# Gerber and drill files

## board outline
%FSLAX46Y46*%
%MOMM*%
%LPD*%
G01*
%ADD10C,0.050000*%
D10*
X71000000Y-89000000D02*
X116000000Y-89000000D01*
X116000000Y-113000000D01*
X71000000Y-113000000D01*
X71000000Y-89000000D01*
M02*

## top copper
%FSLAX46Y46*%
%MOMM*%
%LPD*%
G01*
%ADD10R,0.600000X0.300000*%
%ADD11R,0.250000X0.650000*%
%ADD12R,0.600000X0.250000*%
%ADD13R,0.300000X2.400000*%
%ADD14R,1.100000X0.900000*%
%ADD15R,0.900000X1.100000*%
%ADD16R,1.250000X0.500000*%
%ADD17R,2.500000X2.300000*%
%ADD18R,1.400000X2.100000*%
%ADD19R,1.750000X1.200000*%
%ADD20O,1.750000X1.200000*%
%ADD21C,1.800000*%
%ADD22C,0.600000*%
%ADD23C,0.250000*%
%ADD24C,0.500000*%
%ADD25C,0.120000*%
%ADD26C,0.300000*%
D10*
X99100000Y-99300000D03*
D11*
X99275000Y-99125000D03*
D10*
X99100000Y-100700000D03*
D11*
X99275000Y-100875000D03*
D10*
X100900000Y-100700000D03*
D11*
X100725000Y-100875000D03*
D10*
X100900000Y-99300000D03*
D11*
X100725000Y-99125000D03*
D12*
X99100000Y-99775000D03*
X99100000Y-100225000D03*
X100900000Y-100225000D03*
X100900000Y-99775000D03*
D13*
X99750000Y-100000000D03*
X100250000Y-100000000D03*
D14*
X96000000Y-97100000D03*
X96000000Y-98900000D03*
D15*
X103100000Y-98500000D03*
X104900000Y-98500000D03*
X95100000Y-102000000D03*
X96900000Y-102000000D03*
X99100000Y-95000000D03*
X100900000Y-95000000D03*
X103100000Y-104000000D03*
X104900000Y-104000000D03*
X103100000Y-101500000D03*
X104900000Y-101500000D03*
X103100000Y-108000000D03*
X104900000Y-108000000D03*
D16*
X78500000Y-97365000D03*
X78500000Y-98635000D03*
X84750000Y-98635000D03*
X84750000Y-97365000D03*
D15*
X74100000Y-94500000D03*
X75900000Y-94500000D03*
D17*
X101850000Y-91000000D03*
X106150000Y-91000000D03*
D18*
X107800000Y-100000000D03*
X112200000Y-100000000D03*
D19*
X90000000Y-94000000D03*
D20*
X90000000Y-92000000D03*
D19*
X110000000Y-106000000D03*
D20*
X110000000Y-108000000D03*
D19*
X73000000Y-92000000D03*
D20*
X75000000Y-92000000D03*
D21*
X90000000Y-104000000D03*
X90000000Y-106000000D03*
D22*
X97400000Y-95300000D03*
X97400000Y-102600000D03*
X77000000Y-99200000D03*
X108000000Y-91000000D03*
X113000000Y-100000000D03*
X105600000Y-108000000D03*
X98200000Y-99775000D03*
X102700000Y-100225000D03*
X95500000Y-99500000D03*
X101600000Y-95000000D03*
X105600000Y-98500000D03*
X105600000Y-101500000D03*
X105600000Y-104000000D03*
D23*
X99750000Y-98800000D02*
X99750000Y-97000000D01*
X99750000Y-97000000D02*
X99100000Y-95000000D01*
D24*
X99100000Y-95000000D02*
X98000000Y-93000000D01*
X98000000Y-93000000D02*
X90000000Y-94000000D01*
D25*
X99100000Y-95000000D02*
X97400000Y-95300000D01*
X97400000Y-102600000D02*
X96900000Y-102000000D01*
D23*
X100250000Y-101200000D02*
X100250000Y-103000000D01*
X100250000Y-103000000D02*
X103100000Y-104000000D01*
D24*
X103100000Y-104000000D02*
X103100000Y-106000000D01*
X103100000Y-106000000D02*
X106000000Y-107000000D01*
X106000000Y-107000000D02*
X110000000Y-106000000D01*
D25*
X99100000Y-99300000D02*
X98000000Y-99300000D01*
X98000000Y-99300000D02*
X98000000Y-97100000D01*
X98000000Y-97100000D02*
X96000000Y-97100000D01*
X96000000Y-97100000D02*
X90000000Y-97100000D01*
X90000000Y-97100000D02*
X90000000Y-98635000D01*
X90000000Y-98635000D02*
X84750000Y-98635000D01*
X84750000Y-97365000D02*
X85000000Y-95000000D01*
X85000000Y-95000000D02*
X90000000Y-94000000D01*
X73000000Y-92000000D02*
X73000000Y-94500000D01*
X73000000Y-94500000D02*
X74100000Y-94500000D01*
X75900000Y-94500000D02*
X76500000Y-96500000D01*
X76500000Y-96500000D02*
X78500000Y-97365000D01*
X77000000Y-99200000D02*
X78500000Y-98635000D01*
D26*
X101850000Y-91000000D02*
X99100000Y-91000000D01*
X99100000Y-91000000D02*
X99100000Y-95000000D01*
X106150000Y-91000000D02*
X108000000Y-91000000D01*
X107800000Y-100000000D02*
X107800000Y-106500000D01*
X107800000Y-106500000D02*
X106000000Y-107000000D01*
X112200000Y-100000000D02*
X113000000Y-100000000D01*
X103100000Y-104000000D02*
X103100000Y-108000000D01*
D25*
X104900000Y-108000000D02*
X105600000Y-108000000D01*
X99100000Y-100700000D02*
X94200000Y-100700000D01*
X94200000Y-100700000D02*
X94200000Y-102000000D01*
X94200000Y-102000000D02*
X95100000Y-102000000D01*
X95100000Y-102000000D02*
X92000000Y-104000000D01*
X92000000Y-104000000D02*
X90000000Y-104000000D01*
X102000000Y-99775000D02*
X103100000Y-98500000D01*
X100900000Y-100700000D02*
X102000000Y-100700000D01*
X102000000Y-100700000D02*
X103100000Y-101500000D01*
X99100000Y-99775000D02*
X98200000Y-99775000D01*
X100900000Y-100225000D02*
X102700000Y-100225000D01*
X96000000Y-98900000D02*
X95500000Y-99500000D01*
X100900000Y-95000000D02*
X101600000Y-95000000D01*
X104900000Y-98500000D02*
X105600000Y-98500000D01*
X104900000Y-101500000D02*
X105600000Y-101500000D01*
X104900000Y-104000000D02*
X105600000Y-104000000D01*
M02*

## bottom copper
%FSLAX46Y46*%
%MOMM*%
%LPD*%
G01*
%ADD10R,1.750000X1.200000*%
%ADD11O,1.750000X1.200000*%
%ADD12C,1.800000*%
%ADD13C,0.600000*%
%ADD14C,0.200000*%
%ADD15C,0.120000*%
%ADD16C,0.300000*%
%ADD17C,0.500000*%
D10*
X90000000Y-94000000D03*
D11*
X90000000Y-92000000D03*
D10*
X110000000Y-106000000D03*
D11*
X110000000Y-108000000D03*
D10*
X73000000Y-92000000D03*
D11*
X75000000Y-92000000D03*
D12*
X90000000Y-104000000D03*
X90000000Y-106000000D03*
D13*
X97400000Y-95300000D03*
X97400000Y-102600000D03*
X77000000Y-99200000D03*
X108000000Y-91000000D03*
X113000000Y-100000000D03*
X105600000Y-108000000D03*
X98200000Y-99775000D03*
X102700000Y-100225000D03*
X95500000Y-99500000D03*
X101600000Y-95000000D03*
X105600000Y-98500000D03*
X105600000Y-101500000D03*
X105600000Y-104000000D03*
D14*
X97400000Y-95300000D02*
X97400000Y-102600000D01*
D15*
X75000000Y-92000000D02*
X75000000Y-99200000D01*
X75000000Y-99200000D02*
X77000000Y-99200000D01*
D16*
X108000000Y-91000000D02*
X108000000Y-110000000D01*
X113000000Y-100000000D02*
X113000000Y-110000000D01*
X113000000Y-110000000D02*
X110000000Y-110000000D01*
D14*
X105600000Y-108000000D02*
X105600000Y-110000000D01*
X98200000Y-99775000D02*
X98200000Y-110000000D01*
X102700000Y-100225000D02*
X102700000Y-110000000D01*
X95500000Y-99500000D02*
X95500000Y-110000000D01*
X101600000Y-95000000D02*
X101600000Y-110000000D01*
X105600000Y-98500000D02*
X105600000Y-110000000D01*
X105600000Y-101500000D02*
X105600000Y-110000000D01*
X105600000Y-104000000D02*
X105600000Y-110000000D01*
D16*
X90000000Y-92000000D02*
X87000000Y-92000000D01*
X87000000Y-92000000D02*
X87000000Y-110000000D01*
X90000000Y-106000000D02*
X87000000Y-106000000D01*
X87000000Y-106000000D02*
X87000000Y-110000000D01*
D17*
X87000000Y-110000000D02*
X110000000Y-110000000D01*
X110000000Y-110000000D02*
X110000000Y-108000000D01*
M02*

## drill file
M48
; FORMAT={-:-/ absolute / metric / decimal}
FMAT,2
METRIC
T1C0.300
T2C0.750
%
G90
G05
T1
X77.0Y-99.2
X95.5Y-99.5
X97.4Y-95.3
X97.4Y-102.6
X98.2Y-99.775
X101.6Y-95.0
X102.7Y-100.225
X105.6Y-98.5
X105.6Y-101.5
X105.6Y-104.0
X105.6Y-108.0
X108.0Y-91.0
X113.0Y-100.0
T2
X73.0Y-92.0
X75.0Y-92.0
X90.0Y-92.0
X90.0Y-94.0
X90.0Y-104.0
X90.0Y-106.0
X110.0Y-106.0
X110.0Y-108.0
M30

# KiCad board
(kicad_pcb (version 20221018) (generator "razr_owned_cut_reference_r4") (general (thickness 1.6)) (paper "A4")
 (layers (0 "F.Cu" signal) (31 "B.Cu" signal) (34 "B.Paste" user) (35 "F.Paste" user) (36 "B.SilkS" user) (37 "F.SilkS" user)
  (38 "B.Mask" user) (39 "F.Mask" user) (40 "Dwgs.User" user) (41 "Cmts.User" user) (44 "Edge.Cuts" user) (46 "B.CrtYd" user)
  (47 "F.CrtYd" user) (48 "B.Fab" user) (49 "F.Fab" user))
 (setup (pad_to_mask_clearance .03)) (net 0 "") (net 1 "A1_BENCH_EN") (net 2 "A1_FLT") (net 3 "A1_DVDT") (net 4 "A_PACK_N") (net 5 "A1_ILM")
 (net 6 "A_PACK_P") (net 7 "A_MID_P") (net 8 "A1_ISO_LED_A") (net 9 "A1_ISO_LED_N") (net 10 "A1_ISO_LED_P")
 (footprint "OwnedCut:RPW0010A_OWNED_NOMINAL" (layer "F.Cu") (at 100 100)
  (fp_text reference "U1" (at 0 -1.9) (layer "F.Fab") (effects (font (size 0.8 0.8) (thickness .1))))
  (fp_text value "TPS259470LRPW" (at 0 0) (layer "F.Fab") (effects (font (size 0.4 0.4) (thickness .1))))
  (pad "1" smd rect (at -0.9 -0.7) (size 0.6 0.3) (layers "F.Cu" "F.Paste" "F.Mask") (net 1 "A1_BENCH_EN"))
  (pad "1" smd rect (at -0.725 -0.875) (size 0.25 0.65) (layers "F.Cu" "F.Paste" "F.Mask") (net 1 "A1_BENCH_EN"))
  (pad "4" smd rect (at -0.9 0.7) (size 0.6 0.3) (layers "F.Cu" "F.Paste" "F.Mask") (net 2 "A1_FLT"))
  (pad "4" smd rect (at -0.725 0.875) (size 0.25 0.65) (layers "F.Cu" "F.Paste" "F.Mask") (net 2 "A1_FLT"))
  (pad "7" smd rect (at 0.9 0.7) (size 0.6 0.3) (layers "F.Cu" "F.Paste" "F.Mask") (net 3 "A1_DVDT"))
  (pad "7" smd rect (at 0.725 0.875) (size 0.25 0.65) (layers "F.Cu" "F.Paste" "F.Mask") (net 3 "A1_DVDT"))
  (pad "10" smd rect (at 0.9 -0.7) (size 0.6 0.3) (layers "F.Cu" "F.Paste" "F.Mask"))
  (pad "10" smd rect (at 0.725 -0.875) (size 0.25 0.65) (layers "F.Cu" "F.Paste" "F.Mask"))
  (pad "2" smd rect (at -0.9 -0.225) (size 0.6 0.25) (layers "F.Cu" "F.Paste" "F.Mask") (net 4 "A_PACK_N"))
  (pad "3" smd rect (at -0.9 0.225) (size 0.6 0.25) (layers "F.Cu" "F.Paste" "F.Mask"))
  (pad "8" smd rect (at 0.9 0.225) (size 0.6 0.25) (layers "F.Cu" "F.Paste" "F.Mask") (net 4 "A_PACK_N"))
  (pad "9" smd rect (at 0.9 -0.225) (size 0.6 0.25) (layers "F.Cu" "F.Paste" "F.Mask") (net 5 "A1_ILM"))
  (pad "5" smd rect (at -0.25 0) (size 0.3 2.4) (layers "F.Cu" "F.Paste" "F.Mask") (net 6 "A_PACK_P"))
  (pad "6" smd rect (at 0.25 0) (size 0.3 2.4) (layers "F.Cu" "F.Paste" "F.Mask") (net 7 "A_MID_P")))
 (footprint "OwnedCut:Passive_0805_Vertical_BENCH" (layer "F.Cu") (at 96 98)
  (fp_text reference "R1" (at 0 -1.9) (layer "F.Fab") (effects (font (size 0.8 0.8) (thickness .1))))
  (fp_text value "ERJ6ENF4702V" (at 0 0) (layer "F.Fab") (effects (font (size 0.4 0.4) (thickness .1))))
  (pad "1" smd rect (at 0 -0.9) (size 1.1 0.9) (layers "F.Cu" "F.Paste" "F.Mask") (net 1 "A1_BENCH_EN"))
  (pad "2" smd rect (at 0 0.9) (size 1.1 0.9) (layers "F.Cu" "F.Paste" "F.Mask") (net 4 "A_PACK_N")))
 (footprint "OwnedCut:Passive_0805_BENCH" (layer "F.Cu") (at 104 98.5)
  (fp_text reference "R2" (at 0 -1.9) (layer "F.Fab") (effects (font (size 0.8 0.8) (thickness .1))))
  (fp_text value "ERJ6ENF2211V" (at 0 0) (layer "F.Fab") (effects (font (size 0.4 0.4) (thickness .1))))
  (pad "1" smd rect (at -0.9 0) (size 0.9 1.1) (layers "F.Cu" "F.Paste" "F.Mask") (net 5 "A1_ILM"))
  (pad "2" smd rect (at 0.9 0) (size 0.9 1.1) (layers "F.Cu" "F.Paste" "F.Mask") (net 4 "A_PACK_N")))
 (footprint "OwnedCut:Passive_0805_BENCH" (layer "F.Cu") (at 96 102)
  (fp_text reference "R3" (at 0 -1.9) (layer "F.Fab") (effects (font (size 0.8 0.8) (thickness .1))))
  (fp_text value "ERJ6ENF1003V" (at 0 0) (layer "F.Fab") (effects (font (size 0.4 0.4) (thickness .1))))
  (pad "1" smd rect (at -0.9 0) (size 0.9 1.1) (layers "F.Cu" "F.Paste" "F.Mask") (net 2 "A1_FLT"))
  (pad "2" smd rect (at 0.9 0) (size 0.9 1.1) (layers "F.Cu" "F.Paste" "F.Mask") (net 6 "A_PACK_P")))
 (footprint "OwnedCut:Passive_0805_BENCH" (layer "F.Cu") (at 100 95)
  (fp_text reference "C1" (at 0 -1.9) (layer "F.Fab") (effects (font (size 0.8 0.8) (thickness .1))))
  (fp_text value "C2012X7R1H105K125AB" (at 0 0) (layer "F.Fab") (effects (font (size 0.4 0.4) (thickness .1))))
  (pad "1" smd rect (at -0.9 0) (size 0.9 1.1) (layers "F.Cu" "F.Paste" "F.Mask") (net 6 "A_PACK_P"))
  (pad "2" smd rect (at 0.9 0) (size 0.9 1.1) (layers "F.Cu" "F.Paste" "F.Mask") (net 4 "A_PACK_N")))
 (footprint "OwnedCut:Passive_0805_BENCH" (layer "F.Cu") (at 104 104)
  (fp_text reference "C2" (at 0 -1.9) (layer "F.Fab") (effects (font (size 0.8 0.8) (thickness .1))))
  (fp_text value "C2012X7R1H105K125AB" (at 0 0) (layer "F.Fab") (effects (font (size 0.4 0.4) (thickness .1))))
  (pad "1" smd rect (at -0.9 0) (size 0.9 1.1) (layers "F.Cu" "F.Paste" "F.Mask") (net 7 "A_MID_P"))
  (pad "2" smd rect (at 0.9 0) (size 0.9 1.1) (layers "F.Cu" "F.Paste" "F.Mask") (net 4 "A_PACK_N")))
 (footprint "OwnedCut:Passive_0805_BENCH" (layer "F.Cu") (at 104 101.5)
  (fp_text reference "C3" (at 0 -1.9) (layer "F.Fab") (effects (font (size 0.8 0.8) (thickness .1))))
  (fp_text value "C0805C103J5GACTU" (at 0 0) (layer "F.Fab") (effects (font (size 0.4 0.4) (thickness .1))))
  (pad "1" smd rect (at -0.9 0) (size 0.9 1.1) (layers "F.Cu" "F.Paste" "F.Mask") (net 3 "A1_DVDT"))
  (pad "2" smd rect (at 0.9 0) (size 0.9 1.1) (layers "F.Cu" "F.Paste" "F.Mask") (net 4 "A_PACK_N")))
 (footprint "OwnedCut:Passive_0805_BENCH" (layer "F.Cu") (at 104 108)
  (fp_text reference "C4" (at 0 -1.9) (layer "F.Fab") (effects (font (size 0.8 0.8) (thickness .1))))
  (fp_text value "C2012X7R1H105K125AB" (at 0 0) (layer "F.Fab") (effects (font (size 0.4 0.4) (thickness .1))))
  (pad "1" smd rect (at -0.9 0) (size 0.9 1.1) (layers "F.Cu" "F.Paste" "F.Mask") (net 7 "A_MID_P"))
  (pad "2" smd rect (at 0.9 0) (size 0.9 1.1) (layers "F.Cu" "F.Paste" "F.Mask") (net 4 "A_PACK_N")))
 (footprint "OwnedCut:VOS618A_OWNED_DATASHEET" (layer "F.Cu") (at 81.625 98)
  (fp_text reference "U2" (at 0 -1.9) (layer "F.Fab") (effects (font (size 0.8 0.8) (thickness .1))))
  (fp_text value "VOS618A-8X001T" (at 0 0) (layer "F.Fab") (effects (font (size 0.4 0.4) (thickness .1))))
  (pad "1" smd rect (at -3.125 -0.635) (size 1.25 0.5) (layers "F.Cu" "F.Paste" "F.Mask") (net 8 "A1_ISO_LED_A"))
  (pad "2" smd rect (at -3.125 0.635) (size 1.25 0.5) (layers "F.Cu" "F.Paste" "F.Mask") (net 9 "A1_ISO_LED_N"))
  (pad "3" smd rect (at 3.125 0.635) (size 1.25 0.5) (layers "F.Cu" "F.Paste" "F.Mask") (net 1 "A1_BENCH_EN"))
  (pad "4" smd rect (at 3.125 -0.635) (size 1.25 0.5) (layers "F.Cu" "F.Paste" "F.Mask") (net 6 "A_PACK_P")))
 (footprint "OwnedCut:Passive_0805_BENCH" (layer "F.Cu") (at 75 94.5)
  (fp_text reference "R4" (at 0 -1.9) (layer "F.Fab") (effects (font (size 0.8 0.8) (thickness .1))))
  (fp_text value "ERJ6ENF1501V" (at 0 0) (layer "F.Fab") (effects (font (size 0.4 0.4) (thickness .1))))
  (pad "1" smd rect (at -0.9 0) (size 0.9 1.1) (layers "F.Cu" "F.Paste" "F.Mask") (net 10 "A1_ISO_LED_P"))
  (pad "2" smd rect (at 0.9 0) (size 0.9 1.1) (layers "F.Cu" "F.Paste" "F.Mask") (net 8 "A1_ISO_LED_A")))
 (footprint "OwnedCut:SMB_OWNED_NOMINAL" (layer "F.Cu") (at 104 91)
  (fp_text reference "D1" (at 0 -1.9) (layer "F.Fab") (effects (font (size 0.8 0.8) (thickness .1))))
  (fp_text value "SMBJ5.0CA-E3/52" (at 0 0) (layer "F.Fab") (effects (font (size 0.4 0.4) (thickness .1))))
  (pad "1" smd rect (at -2.15 0) (size 2.5 2.3) (layers "F.Cu" "F.Paste" "F.Mask") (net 6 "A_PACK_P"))
  (pad "2" smd rect (at 2.15 0) (size 2.5 2.3) (layers "F.Cu" "F.Paste" "F.Mask") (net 4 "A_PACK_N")))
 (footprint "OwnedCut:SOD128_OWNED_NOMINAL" (layer "F.Cu") (at 110 100)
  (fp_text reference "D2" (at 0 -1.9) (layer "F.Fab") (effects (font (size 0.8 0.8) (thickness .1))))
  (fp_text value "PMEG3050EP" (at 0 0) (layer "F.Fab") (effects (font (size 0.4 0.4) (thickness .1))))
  (pad "1" smd rect (at -2.2 0) (size 1.4 2.1) (layers "F.Cu" "F.Paste" "F.Mask") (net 7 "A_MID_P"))
  (pad "2" smd rect (at 2.2 0) (size 1.4 2.1) (layers "F.Cu" "F.Paste" "F.Mask") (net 4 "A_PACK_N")))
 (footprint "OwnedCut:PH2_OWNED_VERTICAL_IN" (layer "F.Cu") (at 90 94)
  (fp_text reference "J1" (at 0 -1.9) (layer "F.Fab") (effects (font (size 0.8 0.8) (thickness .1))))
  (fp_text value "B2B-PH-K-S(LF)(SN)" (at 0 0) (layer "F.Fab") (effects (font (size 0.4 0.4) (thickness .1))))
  (pad "1" thru_hole rect (at 0 0) (size 1.75 1.2) (drill .75) (layers "*.Cu" "*.Mask") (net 6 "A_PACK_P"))
  (pad "2" thru_hole oval (at 0 -2) (size 1.75 1.2) (drill .75) (layers "*.Cu" "*.Mask") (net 4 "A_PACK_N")))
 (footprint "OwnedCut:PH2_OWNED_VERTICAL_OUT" (layer "F.Cu") (at 110 106)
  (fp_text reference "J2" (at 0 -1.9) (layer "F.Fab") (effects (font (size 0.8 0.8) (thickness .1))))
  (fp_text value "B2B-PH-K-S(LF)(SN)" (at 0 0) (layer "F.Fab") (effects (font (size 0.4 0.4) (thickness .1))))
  (pad "1" thru_hole rect (at 0 0) (size 1.75 1.2) (drill .75) (layers "*.Cu" "*.Mask") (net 7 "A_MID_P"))
  (pad "2" thru_hole oval (at 0 2) (size 1.75 1.2) (drill .75) (layers "*.Cu" "*.Mask") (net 4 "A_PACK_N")))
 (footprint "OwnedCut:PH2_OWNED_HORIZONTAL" (layer "F.Cu") (at 73 92)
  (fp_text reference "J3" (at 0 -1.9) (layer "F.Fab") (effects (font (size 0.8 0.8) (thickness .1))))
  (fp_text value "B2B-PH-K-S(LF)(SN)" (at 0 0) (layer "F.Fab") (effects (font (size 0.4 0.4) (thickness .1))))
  (pad "1" thru_hole rect (at 0 0) (size 1.75 1.2) (drill .75) (layers "*.Cu" "*.Mask") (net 10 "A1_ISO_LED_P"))
  (pad "2" thru_hole oval (at 2 0) (size 1.75 1.2) (drill .75) (layers "*.Cu" "*.Mask") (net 9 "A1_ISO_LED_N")))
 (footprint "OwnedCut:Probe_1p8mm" (layer "F.Cu") (at 90 104)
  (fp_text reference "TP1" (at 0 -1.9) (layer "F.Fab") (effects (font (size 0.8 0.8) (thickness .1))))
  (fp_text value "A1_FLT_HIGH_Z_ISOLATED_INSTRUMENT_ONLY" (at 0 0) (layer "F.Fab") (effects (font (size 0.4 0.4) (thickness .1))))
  (pad "1" thru_hole circle (at 0 0) (size 1.8 1.8) (drill .75) (layers "*.Cu" "*.Mask") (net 2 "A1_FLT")))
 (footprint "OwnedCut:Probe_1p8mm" (layer "F.Cu") (at 90 106)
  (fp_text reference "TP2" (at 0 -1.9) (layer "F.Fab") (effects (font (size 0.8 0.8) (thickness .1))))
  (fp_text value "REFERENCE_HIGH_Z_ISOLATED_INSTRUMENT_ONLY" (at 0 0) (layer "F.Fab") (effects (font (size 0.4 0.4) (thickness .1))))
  (pad "1" thru_hole circle (at 0 0) (size 1.8 1.8) (drill .75) (layers "*.Cu" "*.Mask") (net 4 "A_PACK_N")))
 (segment (start 99.75 98.8) (end 99.75 97) (width 0.25) (layer "F.Cu") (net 6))
 (segment (start 99.75 97) (end 99.1 95) (width 0.25) (layer "F.Cu") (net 6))
 (segment (start 99.1 95) (end 98 93) (width 0.5) (layer "F.Cu") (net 6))
 (segment (start 98 93) (end 90 94) (width 0.5) (layer "F.Cu") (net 6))
 (segment (start 99.1 95) (end 97.4 95.3) (width 0.12) (layer "F.Cu") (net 6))
 (via (at 97.4 95.3) (size .6) (drill .3) (layers "F.Cu" "B.Cu") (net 6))
 (segment (start 97.4 95.3) (end 97.4 102.6) (width 0.2) (layer "B.Cu") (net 6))
 (via (at 97.4 102.6) (size .6) (drill .3) (layers "F.Cu" "B.Cu") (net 6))
 (segment (start 97.4 102.6) (end 96.9 102) (width 0.12) (layer "F.Cu") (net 6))
 (segment (start 100.25 101.2) (end 100.25 103) (width 0.25) (layer "F.Cu") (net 7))
 (segment (start 100.25 103) (end 103.1 104) (width 0.25) (layer "F.Cu") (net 7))
 (segment (start 103.1 104) (end 103.1 106) (width 0.5) (layer "F.Cu") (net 7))
 (segment (start 103.1 106) (end 106 107) (width 0.5) (layer "F.Cu") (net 7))
 (segment (start 106 107) (end 110 106) (width 0.5) (layer "F.Cu") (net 7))
 (segment (start 99.1 99.3) (end 98 99.3) (width 0.12) (layer "F.Cu") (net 1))
 (segment (start 98 99.3) (end 98 97.1) (width 0.12) (layer "F.Cu") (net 1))
 (segment (start 98 97.1) (end 96 97.1) (width 0.12) (layer "F.Cu") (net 1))
 (segment (start 96 97.1) (end 90 97.1) (width 0.12) (layer "F.Cu") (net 1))
 (segment (start 90 97.1) (end 90 98.635) (width 0.12) (layer "F.Cu") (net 1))
 (segment (start 90 98.635) (end 84.75 98.635) (width 0.12) (layer "F.Cu") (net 1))
 (segment (start 84.75 97.365) (end 85 95) (width 0.12) (layer "F.Cu") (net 6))
 (segment (start 85 95) (end 90 94) (width 0.12) (layer "F.Cu") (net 6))
 (segment (start 73 92) (end 73 94.5) (width 0.12) (layer "F.Cu") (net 10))
 (segment (start 73 94.5) (end 74.1 94.5) (width 0.12) (layer "F.Cu") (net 10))
 (segment (start 75.9 94.5) (end 76.5 96.5) (width 0.12) (layer "F.Cu") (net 8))
 (segment (start 76.5 96.5) (end 78.5 97.365) (width 0.12) (layer "F.Cu") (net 8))
 (segment (start 75 92) (end 75 99.2) (width 0.12) (layer "B.Cu") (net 9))
 (segment (start 75 99.2) (end 77 99.2) (width 0.12) (layer "B.Cu") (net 9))
 (via (at 77 99.2) (size .6) (drill .3) (layers "F.Cu" "B.Cu") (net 9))
 (segment (start 77 99.2) (end 78.5 98.635) (width 0.12) (layer "F.Cu") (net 9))
 (segment (start 101.85 91) (end 99.1 91) (width 0.3) (layer "F.Cu") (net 6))
 (segment (start 99.1 91) (end 99.1 95) (width 0.3) (layer "F.Cu") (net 6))
 (segment (start 106.15 91) (end 108 91) (width 0.3) (layer "F.Cu") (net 4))
 (via (at 108 91) (size .6) (drill .3) (layers "F.Cu" "B.Cu") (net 4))
 (segment (start 108 91) (end 108 110) (width 0.3) (layer "B.Cu") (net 4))
 (segment (start 107.8 100) (end 107.8 106.5) (width 0.3) (layer "F.Cu") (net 7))
 (segment (start 107.8 106.5) (end 106 107) (width 0.3) (layer "F.Cu") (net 7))
 (segment (start 112.2 100) (end 113 100) (width 0.3) (layer "F.Cu") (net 4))
 (via (at 113 100) (size .6) (drill .3) (layers "F.Cu" "B.Cu") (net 4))
 (segment (start 113 100) (end 113 110) (width 0.3) (layer "B.Cu") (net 4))
 (segment (start 113 110) (end 110 110) (width 0.3) (layer "B.Cu") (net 4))
 (segment (start 103.1 104) (end 103.1 108) (width 0.3) (layer "F.Cu") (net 7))
 (segment (start 104.9 108) (end 105.6 108) (width 0.12) (layer "F.Cu") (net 4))
 (via (at 105.6 108) (size .6) (drill .3) (layers "F.Cu" "B.Cu") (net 4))
 (segment (start 105.6 108) (end 105.6 110) (width 0.2) (layer "B.Cu") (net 4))
 (segment (start 99.1 100.7) (end 94.2 100.7) (width 0.12) (layer "F.Cu") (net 2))
 (segment (start 94.2 100.7) (end 94.2 102) (width 0.12) (layer "F.Cu") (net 2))
 (segment (start 94.2 102) (end 95.1 102) (width 0.12) (layer "F.Cu") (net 2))
 (segment (start 95.1 102) (end 92 104) (width 0.12) (layer "F.Cu") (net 2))
 (segment (start 92 104) (end 90 104) (width 0.12) (layer "F.Cu") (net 2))
 (segment (start 102 99.775) (end 103.1 98.5) (width 0.12) (layer "F.Cu") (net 5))
 (segment (start 100.9 100.7) (end 102 100.7) (width 0.12) (layer "F.Cu") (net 3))
 (segment (start 102 100.7) (end 103.1 101.5) (width 0.12) (layer "F.Cu") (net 3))
 (segment (start 99.1 99.775) (end 98.2 99.775) (width 0.12) (layer "F.Cu") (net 4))
 (via (at 98.2 99.775) (size .6) (drill .3) (layers "F.Cu" "B.Cu") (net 4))
 (segment (start 98.2 99.775) (end 98.2 110) (width 0.2) (layer "B.Cu") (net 4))
 (segment (start 100.9 100.225) (end 102.7 100.225) (width 0.12) (layer "F.Cu") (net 4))
 (via (at 102.7 100.225) (size .6) (drill .3) (layers "F.Cu" "B.Cu") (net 4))
 (segment (start 102.7 100.225) (end 102.7 110) (width 0.2) (layer "B.Cu") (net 4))
 (segment (start 96 98.9) (end 95.5 99.5) (width 0.12) (layer "F.Cu") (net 4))
 (via (at 95.5 99.5) (size .6) (drill .3) (layers "F.Cu" "B.Cu") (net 4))
 (segment (start 95.5 99.5) (end 95.5 110) (width 0.2) (layer "B.Cu") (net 4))
 (segment (start 100.9 95) (end 101.6 95) (width 0.12) (layer "F.Cu") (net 4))
 (via (at 101.6 95) (size .6) (drill .3) (layers "F.Cu" "B.Cu") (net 4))
 (segment (start 101.6 95) (end 101.6 110) (width 0.2) (layer "B.Cu") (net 4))
 (segment (start 104.9 98.5) (end 105.6 98.5) (width 0.12) (layer "F.Cu") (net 4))
 (via (at 105.6 98.5) (size .6) (drill .3) (layers "F.Cu" "B.Cu") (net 4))
 (segment (start 105.6 98.5) (end 105.6 110) (width 0.2) (layer "B.Cu") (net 4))
 (segment (start 104.9 101.5) (end 105.6 101.5) (width 0.12) (layer "F.Cu") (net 4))
 (via (at 105.6 101.5) (size .6) (drill .3) (layers "F.Cu" "B.Cu") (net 4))
 (segment (start 105.6 101.5) (end 105.6 110) (width 0.2) (layer "B.Cu") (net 4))
 (segment (start 104.9 104) (end 105.6 104) (width 0.12) (layer "F.Cu") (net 4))
 (via (at 105.6 104) (size .6) (drill .3) (layers "F.Cu" "B.Cu") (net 4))
 (segment (start 105.6 104) (end 105.6 110) (width 0.2) (layer "B.Cu") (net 4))
 (segment (start 90 92) (end 87 92) (width 0.3) (layer "B.Cu") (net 4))
 (segment (start 87 92) (end 87 110) (width 0.3) (layer "B.Cu") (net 4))
 (segment (start 90 106) (end 87 106) (width 0.3) (layer "B.Cu") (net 4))
 (segment (start 87 106) (end 87 110) (width 0.3) (layer "B.Cu") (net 4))
 (segment (start 87 110) (end 110 110) (width 0.5) (layer "B.Cu") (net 4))
 (segment (start 110 110) (end 110 108) (width 0.5) (layer "B.Cu") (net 4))
 (gr_rect (start 71 89) (end 116 113) (stroke (width .05) (type default)) (fill none) (layer "Edge.Cuts")))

